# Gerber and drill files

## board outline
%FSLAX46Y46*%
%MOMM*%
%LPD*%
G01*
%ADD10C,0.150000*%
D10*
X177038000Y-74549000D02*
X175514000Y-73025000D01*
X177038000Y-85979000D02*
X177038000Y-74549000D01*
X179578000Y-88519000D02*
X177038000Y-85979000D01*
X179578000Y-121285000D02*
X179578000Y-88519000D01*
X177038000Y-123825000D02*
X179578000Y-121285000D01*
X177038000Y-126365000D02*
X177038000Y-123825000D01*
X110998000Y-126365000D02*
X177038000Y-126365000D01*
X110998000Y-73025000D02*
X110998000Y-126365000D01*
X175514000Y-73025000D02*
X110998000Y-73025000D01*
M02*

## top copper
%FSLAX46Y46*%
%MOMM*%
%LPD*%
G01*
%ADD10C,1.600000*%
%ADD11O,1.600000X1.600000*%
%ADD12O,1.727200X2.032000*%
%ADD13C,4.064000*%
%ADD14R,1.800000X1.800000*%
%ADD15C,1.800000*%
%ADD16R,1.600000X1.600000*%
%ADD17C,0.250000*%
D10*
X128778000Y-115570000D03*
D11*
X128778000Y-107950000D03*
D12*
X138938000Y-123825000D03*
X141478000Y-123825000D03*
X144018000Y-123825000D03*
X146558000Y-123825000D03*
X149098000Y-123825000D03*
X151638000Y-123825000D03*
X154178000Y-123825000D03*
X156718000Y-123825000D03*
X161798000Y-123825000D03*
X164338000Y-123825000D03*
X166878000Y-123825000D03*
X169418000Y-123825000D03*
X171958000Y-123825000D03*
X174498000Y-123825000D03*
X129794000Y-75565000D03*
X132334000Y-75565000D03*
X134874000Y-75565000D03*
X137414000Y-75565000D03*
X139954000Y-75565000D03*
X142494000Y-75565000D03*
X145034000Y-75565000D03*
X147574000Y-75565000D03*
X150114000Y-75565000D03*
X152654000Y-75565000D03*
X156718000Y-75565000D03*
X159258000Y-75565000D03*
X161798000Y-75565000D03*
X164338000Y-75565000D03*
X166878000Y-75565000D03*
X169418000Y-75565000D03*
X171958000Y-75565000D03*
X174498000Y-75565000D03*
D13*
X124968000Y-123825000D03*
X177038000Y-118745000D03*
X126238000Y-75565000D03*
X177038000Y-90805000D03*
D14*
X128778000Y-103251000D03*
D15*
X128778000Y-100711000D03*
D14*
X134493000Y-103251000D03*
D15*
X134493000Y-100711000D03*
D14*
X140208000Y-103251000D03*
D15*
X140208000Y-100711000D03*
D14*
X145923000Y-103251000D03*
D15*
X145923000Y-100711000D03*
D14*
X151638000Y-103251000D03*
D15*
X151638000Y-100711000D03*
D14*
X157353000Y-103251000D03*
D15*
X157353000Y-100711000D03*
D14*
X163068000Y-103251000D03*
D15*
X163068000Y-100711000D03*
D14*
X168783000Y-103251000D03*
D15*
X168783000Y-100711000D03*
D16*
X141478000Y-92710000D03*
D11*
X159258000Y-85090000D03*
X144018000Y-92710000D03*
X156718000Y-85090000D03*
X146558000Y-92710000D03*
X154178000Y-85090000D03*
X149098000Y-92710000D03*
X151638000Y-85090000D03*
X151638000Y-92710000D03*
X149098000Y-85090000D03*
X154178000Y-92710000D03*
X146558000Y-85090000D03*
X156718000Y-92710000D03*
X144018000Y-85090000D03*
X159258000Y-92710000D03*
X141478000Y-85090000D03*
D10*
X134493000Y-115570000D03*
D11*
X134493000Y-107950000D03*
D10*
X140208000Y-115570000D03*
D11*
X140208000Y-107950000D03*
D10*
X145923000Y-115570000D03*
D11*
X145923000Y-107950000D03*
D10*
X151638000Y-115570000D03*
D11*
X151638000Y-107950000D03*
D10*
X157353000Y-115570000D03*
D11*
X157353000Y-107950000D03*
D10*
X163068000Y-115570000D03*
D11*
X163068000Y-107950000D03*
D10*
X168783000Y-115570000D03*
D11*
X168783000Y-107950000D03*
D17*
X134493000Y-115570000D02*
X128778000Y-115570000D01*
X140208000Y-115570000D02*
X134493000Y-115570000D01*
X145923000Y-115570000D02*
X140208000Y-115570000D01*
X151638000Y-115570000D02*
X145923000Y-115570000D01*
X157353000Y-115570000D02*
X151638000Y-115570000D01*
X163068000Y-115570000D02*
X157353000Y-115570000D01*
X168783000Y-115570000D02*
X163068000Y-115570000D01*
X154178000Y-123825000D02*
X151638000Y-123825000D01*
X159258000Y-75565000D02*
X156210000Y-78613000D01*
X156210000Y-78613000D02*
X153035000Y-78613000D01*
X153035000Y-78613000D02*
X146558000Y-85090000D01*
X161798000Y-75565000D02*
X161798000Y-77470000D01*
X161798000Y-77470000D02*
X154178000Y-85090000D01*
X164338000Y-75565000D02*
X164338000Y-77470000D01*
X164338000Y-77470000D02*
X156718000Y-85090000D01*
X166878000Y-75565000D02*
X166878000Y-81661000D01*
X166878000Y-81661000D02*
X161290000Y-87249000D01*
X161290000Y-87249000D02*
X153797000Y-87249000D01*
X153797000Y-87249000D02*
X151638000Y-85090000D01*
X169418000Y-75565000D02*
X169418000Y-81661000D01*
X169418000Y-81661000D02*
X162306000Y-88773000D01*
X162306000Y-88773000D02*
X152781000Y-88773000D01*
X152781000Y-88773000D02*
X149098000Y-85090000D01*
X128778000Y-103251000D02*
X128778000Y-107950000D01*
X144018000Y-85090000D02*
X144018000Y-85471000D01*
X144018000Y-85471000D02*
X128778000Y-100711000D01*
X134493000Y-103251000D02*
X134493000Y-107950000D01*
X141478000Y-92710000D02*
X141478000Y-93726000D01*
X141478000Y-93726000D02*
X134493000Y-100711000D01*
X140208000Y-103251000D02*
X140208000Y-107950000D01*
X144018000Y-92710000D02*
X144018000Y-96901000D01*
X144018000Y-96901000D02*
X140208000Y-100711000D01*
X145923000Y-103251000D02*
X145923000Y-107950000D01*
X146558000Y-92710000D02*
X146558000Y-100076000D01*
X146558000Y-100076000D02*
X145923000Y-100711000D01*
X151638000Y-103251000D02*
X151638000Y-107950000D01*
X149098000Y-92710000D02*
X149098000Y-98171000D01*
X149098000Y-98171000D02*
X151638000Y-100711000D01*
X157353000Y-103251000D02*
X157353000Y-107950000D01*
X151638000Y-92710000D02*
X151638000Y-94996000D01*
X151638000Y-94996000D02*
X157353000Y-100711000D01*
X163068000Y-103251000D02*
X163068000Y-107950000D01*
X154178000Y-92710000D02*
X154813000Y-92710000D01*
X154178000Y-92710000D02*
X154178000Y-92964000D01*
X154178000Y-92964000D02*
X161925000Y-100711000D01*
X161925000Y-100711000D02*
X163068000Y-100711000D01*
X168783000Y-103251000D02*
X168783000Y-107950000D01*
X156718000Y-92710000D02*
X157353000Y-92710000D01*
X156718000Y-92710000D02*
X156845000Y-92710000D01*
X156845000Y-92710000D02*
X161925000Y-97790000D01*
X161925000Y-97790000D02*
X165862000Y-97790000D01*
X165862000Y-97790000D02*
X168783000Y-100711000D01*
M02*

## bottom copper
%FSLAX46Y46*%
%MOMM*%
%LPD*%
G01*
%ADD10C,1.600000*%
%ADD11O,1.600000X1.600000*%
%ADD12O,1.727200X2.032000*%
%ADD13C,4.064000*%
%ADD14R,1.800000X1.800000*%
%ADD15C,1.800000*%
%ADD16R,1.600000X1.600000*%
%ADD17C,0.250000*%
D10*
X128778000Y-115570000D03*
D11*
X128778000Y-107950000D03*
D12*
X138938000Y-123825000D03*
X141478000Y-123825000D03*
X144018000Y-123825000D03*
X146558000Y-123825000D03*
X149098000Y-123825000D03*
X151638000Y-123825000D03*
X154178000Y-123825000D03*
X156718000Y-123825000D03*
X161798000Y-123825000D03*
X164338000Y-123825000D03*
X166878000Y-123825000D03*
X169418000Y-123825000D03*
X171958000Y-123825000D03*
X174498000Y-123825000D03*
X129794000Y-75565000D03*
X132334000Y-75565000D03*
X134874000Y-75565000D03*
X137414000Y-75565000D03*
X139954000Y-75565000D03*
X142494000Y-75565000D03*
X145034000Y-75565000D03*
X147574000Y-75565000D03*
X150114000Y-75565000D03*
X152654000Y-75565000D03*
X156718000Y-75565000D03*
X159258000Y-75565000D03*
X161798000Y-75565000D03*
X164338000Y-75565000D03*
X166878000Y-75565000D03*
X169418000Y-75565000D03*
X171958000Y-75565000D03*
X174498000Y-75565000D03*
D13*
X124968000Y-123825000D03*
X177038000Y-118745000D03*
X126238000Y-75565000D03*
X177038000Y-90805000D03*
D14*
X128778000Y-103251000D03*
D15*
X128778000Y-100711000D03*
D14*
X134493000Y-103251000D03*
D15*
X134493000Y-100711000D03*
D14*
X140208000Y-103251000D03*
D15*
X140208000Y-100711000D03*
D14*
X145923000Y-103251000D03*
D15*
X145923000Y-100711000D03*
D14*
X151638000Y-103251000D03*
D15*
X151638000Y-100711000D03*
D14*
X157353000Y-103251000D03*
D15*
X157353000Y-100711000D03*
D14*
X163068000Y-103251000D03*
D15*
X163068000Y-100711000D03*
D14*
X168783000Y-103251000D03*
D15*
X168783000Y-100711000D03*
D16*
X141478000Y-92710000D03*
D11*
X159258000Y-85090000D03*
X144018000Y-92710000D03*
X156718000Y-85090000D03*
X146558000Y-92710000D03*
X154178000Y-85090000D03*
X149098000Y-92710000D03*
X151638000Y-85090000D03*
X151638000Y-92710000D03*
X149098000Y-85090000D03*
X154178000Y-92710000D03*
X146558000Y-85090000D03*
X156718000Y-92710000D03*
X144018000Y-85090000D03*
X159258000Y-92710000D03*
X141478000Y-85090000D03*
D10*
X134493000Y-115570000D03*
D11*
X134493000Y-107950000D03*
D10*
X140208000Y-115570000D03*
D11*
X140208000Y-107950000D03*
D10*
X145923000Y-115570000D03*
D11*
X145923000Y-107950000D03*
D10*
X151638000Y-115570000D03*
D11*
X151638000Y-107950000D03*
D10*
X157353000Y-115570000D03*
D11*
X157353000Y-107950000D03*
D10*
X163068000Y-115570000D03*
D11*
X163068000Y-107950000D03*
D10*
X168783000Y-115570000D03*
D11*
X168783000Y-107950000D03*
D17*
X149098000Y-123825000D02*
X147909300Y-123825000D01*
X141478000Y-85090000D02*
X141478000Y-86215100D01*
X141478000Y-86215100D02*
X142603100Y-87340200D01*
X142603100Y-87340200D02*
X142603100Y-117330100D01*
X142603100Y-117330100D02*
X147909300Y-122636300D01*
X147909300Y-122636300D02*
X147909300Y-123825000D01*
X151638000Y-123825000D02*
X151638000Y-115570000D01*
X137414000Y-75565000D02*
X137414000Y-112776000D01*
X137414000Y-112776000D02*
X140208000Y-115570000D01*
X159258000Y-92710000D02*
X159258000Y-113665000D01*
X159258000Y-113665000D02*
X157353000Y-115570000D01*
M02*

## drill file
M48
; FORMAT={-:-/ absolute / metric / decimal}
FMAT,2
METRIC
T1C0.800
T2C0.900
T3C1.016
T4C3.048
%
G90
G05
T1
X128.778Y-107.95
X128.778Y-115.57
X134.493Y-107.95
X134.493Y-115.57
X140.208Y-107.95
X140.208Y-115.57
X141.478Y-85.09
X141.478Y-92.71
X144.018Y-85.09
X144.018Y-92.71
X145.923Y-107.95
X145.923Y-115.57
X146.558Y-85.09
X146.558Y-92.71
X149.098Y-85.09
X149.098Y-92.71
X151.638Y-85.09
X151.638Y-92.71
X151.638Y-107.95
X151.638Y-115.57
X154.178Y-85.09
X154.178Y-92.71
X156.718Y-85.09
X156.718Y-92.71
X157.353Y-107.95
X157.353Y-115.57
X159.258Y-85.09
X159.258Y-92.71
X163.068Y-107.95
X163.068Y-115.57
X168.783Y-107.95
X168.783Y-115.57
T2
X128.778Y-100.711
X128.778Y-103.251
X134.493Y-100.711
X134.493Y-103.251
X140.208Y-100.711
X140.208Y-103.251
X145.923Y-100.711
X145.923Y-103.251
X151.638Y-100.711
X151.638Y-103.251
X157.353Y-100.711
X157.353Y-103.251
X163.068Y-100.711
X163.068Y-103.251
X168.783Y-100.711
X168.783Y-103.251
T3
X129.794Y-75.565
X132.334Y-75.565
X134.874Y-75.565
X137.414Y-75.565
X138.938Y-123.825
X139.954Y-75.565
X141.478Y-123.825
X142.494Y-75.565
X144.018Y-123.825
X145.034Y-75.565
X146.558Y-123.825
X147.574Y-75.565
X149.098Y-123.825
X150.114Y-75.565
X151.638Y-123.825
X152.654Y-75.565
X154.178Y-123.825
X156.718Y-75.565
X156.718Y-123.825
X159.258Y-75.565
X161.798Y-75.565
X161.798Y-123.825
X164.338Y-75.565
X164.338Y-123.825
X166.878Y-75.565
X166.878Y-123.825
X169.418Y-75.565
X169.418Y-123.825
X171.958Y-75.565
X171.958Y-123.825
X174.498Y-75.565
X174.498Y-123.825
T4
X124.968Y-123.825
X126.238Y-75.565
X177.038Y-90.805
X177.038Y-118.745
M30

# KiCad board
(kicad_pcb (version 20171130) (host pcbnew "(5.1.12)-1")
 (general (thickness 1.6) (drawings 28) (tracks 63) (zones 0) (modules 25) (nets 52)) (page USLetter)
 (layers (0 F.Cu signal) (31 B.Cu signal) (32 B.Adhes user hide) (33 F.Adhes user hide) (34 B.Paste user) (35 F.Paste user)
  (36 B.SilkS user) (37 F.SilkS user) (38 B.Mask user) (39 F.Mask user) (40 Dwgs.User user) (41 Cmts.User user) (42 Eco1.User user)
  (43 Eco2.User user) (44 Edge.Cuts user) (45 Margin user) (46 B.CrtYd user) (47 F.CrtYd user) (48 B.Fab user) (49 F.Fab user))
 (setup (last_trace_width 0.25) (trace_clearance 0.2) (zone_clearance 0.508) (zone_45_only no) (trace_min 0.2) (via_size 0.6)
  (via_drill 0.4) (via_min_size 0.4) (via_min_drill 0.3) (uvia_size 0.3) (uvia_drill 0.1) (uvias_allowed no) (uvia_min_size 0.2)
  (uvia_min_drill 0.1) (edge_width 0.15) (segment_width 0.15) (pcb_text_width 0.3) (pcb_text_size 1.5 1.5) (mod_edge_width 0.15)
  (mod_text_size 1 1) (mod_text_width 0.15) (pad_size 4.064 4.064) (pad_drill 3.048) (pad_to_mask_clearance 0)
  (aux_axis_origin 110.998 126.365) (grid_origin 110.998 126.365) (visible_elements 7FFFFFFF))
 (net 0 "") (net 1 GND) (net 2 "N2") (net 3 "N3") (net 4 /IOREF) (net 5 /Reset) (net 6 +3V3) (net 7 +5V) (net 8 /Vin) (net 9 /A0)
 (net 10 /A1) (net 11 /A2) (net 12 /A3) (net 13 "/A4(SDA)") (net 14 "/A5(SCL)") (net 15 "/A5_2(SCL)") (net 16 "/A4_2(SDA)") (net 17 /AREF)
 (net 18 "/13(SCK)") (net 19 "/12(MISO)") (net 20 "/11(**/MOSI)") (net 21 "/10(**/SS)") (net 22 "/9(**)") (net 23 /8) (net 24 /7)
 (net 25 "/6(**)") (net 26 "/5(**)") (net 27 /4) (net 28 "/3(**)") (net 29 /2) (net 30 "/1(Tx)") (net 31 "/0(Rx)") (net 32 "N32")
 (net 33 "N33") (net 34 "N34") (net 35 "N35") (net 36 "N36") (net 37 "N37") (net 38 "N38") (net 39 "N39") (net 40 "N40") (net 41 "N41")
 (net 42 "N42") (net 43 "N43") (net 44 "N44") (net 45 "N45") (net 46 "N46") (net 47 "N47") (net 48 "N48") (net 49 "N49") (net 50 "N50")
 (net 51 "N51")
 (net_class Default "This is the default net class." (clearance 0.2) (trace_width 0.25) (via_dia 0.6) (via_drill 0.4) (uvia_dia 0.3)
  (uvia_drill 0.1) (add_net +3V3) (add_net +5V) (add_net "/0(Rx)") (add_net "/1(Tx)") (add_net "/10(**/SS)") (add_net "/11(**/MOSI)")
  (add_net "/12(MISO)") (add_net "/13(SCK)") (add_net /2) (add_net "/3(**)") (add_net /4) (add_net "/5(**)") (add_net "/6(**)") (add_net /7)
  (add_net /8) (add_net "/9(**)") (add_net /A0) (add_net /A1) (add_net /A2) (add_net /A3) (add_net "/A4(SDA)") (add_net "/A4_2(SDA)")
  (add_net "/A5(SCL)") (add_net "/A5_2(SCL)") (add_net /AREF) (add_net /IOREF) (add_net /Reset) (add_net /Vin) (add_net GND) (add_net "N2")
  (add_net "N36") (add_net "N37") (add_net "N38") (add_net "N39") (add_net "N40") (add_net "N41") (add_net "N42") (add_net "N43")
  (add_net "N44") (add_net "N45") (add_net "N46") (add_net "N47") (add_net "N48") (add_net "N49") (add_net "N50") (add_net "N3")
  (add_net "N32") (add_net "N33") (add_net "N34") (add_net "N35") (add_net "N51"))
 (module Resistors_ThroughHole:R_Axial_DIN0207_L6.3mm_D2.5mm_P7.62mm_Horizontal (layer F.Cu) (at 128.778 115.57 90)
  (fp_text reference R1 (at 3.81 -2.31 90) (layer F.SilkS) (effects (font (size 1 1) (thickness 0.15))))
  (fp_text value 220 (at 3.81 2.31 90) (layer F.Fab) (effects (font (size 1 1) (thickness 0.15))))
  (pad 1 thru_hole circle (at 0 0 90) (size 1.6 1.6) (drill 0.8) (layers *.Cu *.Mask) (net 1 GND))
  (pad 2 thru_hole oval (at 7.62 0 90) (size 1.6 1.6) (drill 0.8) (layers *.Cu *.Mask) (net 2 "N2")))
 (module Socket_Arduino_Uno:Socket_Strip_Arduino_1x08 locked (layer F.Cu) (at 138.938 123.825)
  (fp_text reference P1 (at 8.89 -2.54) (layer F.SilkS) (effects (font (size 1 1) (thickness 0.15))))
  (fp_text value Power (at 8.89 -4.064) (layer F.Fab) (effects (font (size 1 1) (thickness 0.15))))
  (pad 1 thru_hole oval (at 0 0) (size 1.7272 2.032) (drill 1.016) (layers *.Cu *.Mask F.SilkS) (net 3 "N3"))
  (pad 2 thru_hole oval (at 2.54 0) (size 1.7272 2.032) (drill 1.016) (layers *.Cu *.Mask F.SilkS) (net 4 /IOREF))
  (pad 3 thru_hole oval (at 5.08 0) (size 1.7272 2.032) (drill 1.016) (layers *.Cu *.Mask F.SilkS) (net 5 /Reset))
  (pad 4 thru_hole oval (at 7.62 0) (size 1.7272 2.032) (drill 1.016) (layers *.Cu *.Mask F.SilkS) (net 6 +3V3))
  (pad 5 thru_hole oval (at 10.16 0) (size 1.7272 2.032) (drill 1.016) (layers *.Cu *.Mask F.SilkS) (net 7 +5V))
  (pad 6 thru_hole oval (at 12.7 0) (size 1.7272 2.032) (drill 1.016) (layers *.Cu *.Mask F.SilkS) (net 1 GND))
  (pad 7 thru_hole oval (at 15.24 0) (size 1.7272 2.032) (drill 1.016) (layers *.Cu *.Mask F.SilkS) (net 1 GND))
  (pad 8 thru_hole oval (at 17.78 0) (size 1.7272 2.032) (drill 1.016) (layers *.Cu *.Mask F.SilkS) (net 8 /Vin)))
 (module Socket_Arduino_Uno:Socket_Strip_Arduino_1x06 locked (layer F.Cu) (at 161.798 123.825)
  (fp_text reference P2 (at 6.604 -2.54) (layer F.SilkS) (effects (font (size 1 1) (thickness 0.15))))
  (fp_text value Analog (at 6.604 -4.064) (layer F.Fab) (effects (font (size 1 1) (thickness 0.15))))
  (pad 1 thru_hole oval (at 0 0) (size 1.7272 2.032) (drill 1.016) (layers *.Cu *.Mask F.SilkS) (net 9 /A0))
  (pad 2 thru_hole oval (at 2.54 0) (size 1.7272 2.032) (drill 1.016) (layers *.Cu *.Mask F.SilkS) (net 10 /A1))
  (pad 3 thru_hole oval (at 5.08 0) (size 1.7272 2.032) (drill 1.016) (layers *.Cu *.Mask F.SilkS) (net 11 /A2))
  (pad 4 thru_hole oval (at 7.62 0) (size 1.7272 2.032) (drill 1.016) (layers *.Cu *.Mask F.SilkS) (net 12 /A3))
  (pad 5 thru_hole oval (at 10.16 0) (size 1.7272 2.032) (drill 1.016) (layers *.Cu *.Mask F.SilkS) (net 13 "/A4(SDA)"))
  (pad 6 thru_hole oval (at 12.7 0) (size 1.7272 2.032) (drill 1.016) (layers *.Cu *.Mask F.SilkS) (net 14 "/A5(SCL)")))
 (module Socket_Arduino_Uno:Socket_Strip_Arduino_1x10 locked (layer F.Cu) (at 129.794 75.565)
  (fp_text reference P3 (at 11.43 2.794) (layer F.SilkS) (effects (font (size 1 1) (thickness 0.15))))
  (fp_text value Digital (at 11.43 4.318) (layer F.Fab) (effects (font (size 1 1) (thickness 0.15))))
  (pad 1 thru_hole oval (at 0 0) (size 1.7272 2.032) (drill 1.016) (layers *.Cu *.Mask F.SilkS) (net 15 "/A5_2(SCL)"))
  (pad 2 thru_hole oval (at 2.54 0) (size 1.7272 2.032) (drill 1.016) (layers *.Cu *.Mask F.SilkS) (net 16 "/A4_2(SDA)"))
  (pad 3 thru_hole oval (at 5.08 0) (size 1.7272 2.032) (drill 1.016) (layers *.Cu *.Mask F.SilkS) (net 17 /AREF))
  (pad 4 thru_hole oval (at 7.62 0) (size 1.7272 2.032) (drill 1.016) (layers *.Cu *.Mask F.SilkS) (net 1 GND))
  (pad 5 thru_hole oval (at 10.16 0) (size 1.7272 2.032) (drill 1.016) (layers *.Cu *.Mask F.SilkS) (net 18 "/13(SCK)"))
  (pad 6 thru_hole oval (at 12.7 0) (size 1.7272 2.032) (drill 1.016) (layers *.Cu *.Mask F.SilkS) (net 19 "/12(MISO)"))
  (pad 7 thru_hole oval (at 15.24 0) (size 1.7272 2.032) (drill 1.016) (layers *.Cu *.Mask F.SilkS) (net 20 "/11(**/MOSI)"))
  (pad 8 thru_hole oval (at 17.78 0) (size 1.7272 2.032) (drill 1.016) (layers *.Cu *.Mask F.SilkS) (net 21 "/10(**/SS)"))
  (pad 9 thru_hole oval (at 20.32 0) (size 1.7272 2.032) (drill 1.016) (layers *.Cu *.Mask F.SilkS) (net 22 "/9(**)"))
  (pad 10 thru_hole oval (at 22.86 0) (size 1.7272 2.032) (drill 1.016) (layers *.Cu *.Mask F.SilkS) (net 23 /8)))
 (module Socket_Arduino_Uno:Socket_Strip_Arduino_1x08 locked (layer F.Cu) (at 156.718 75.565)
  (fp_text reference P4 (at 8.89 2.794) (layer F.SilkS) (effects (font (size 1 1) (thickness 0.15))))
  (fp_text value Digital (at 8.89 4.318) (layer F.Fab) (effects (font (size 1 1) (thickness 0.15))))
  (pad 1 thru_hole oval (at 0 0) (size 1.7272 2.032) (drill 1.016) (layers *.Cu *.Mask F.SilkS) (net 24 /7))
  (pad 2 thru_hole oval (at 2.54 0) (size 1.7272 2.032) (drill 1.016) (layers *.Cu *.Mask F.SilkS) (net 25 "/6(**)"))
  (pad 3 thru_hole oval (at 5.08 0) (size 1.7272 2.032) (drill 1.016) (layers *.Cu *.Mask F.SilkS) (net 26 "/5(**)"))
  (pad 4 thru_hole oval (at 7.62 0) (size 1.7272 2.032) (drill 1.016) (layers *.Cu *.Mask F.SilkS) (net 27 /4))
  (pad 5 thru_hole oval (at 10.16 0) (size 1.7272 2.032) (drill 1.016) (layers *.Cu *.Mask F.SilkS) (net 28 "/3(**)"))
  (pad 6 thru_hole oval (at 12.7 0) (size 1.7272 2.032) (drill 1.016) (layers *.Cu *.Mask F.SilkS) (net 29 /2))
  (pad 7 thru_hole oval (at 15.24 0) (size 1.7272 2.032) (drill 1.016) (layers *.Cu *.Mask F.SilkS) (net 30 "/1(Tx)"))
  (pad 8 thru_hole oval (at 17.78 0) (size 1.7272 2.032) (drill 1.016) (layers *.Cu *.Mask F.SilkS) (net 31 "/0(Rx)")))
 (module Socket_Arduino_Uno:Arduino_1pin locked (layer F.Cu) (at 124.968 123.825)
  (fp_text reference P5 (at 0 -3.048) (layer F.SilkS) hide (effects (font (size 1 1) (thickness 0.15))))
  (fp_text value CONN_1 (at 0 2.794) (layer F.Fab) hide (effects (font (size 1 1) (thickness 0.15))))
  (pad 1 thru_hole circle (at 0 0) (size 4.064 4.064) (drill 3.048) (layers *.Cu *.Mask F.SilkS) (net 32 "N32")))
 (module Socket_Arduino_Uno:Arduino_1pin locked (layer F.Cu) (at 177.038 118.745)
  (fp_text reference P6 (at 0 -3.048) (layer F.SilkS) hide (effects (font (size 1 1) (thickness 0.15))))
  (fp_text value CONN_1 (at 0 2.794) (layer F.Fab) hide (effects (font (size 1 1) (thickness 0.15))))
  (pad 1 thru_hole circle (at 0 0) (size 4.064 4.064) (drill 3.048) (layers *.Cu *.Mask F.SilkS) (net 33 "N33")))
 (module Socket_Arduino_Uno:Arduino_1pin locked (layer F.Cu) (at 126.238 75.565)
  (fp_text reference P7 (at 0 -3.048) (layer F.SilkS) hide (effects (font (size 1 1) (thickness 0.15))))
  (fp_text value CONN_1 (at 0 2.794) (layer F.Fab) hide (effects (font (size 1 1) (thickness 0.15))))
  (pad 1 thru_hole circle (at 0 0) (size 4.064 4.064) (drill 3.048) (layers *.Cu *.Mask F.SilkS) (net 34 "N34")))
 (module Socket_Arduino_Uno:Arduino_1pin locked (layer F.Cu) (at 177.038 90.805)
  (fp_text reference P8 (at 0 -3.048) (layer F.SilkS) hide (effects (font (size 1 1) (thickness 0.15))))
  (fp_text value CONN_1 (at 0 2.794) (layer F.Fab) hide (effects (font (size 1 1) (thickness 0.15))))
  (pad 1 thru_hole circle (at 0 0) (size 4.064 4.064) (drill 3.048) (layers *.Cu *.Mask F.SilkS) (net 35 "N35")))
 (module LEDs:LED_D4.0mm (layer F.Cu) (at 128.778 103.251 90)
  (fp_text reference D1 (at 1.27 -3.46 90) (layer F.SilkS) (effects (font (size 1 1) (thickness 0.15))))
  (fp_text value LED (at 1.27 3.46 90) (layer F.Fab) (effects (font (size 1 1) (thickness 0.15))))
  (pad 1 thru_hole rect (at 0 0 90) (size 1.8 1.8) (drill 0.9) (layers *.Cu *.Mask) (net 2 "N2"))
  (pad 2 thru_hole circle (at 2.54 0 90) (size 1.8 1.8) (drill 0.9) (layers *.Cu *.Mask) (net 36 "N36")))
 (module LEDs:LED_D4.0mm (layer F.Cu) (at 134.493 103.251 90)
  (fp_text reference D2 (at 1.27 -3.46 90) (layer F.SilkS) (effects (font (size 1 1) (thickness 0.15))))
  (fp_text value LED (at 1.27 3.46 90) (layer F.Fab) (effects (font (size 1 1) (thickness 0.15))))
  (pad 1 thru_hole rect (at 0 0 90) (size 1.8 1.8) (drill 0.9) (layers *.Cu *.Mask) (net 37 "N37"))
  (pad 2 thru_hole circle (at 2.54 0 90) (size 1.8 1.8) (drill 0.9) (layers *.Cu *.Mask) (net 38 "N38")))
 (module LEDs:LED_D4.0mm (layer F.Cu) (at 140.208 103.251 90)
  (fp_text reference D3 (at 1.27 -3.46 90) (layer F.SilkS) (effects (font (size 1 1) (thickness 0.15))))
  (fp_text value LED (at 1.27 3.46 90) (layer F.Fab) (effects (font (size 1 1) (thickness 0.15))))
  (pad 1 thru_hole rect (at 0 0 90) (size 1.8 1.8) (drill 0.9) (layers *.Cu *.Mask) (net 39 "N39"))
  (pad 2 thru_hole circle (at 2.54 0 90) (size 1.8 1.8) (drill 0.9) (layers *.Cu *.Mask) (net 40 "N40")))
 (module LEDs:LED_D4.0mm (layer F.Cu) (at 145.923 103.251 90)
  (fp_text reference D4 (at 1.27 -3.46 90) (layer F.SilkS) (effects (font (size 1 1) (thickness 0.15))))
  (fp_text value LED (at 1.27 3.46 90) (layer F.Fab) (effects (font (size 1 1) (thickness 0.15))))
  (pad 1 thru_hole rect (at 0 0 90) (size 1.8 1.8) (drill 0.9) (layers *.Cu *.Mask) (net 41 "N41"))
  (pad 2 thru_hole circle (at 2.54 0 90) (size 1.8 1.8) (drill 0.9) (layers *.Cu *.Mask) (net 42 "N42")))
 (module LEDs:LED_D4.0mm (layer F.Cu) (at 151.638 103.251 90)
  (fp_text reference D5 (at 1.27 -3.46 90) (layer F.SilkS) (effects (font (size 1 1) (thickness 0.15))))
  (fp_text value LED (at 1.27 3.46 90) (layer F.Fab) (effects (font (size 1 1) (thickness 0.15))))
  (pad 1 thru_hole rect (at 0 0 90) (size 1.8 1.8) (drill 0.9) (layers *.Cu *.Mask) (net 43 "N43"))
  (pad 2 thru_hole circle (at 2.54 0 90) (size 1.8 1.8) (drill 0.9) (layers *.Cu *.Mask) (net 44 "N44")))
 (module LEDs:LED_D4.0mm (layer F.Cu) (at 157.353 103.251 90)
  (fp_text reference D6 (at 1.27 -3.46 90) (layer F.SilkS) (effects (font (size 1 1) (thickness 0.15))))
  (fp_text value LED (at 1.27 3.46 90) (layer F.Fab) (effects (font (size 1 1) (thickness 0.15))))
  (pad 1 thru_hole rect (at 0 0 90) (size 1.8 1.8) (drill 0.9) (layers *.Cu *.Mask) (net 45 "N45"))
  (pad 2 thru_hole circle (at 2.54 0 90) (size 1.8 1.8) (drill 0.9) (layers *.Cu *.Mask) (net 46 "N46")))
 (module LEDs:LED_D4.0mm (layer F.Cu) (at 163.068 103.251 90)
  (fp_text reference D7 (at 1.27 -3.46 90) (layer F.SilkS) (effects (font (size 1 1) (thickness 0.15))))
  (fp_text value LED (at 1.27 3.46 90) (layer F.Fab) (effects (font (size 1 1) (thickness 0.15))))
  (pad 1 thru_hole rect (at 0 0 90) (size 1.8 1.8) (drill 0.9) (layers *.Cu *.Mask) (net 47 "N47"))
  (pad 2 thru_hole circle (at 2.54 0 90) (size 1.8 1.8) (drill 0.9) (layers *.Cu *.Mask) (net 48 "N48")))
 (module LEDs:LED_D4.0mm (layer F.Cu) (at 168.783 103.251 90)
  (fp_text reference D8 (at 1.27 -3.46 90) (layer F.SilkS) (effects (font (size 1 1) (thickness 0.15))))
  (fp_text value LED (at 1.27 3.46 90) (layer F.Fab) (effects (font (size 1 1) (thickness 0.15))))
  (pad 1 thru_hole rect (at 0 0 90) (size 1.8 1.8) (drill 0.9) (layers *.Cu *.Mask) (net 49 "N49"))
  (pad 2 thru_hole circle (at 2.54 0 90) (size 1.8 1.8) (drill 0.9) (layers *.Cu *.Mask) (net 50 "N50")))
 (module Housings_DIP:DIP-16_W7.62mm (layer F.Cu) (at 141.478 92.71 90)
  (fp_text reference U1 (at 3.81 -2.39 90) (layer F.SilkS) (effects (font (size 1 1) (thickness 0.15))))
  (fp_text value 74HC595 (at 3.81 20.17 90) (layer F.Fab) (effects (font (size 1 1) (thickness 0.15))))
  (pad 1 thru_hole rect (at 0 0 90) (size 1.6 1.6) (drill 0.8) (layers *.Cu *.Mask) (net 38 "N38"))
  (pad 9 thru_hole oval (at 7.62 17.78 90) (size 1.6 1.6) (drill 0.8) (layers *.Cu *.Mask) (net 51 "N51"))
  (pad 2 thru_hole oval (at 0 2.54 90) (size 1.6 1.6) (drill 0.8) (layers *.Cu *.Mask) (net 40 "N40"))
  (pad 10 thru_hole oval (at 7.62 15.24 90) (size 1.6 1.6) (drill 0.8) (layers *.Cu *.Mask) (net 27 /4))
  (pad 3 thru_hole oval (at 0 5.08 90) (size 1.6 1.6) (drill 0.8) (layers *.Cu *.Mask) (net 42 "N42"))
  (pad 11 thru_hole oval (at 7.62 12.7 90) (size 1.6 1.6) (drill 0.8) (layers *.Cu *.Mask) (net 26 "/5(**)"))
  (pad 4 thru_hole oval (at 0 7.62 90) (size 1.6 1.6) (drill 0.8) (layers *.Cu *.Mask) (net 44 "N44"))
  (pad 12 thru_hole oval (at 7.62 10.16 90) (size 1.6 1.6) (drill 0.8) (layers *.Cu *.Mask) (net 28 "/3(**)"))
  (pad 5 thru_hole oval (at 0 10.16 90) (size 1.6 1.6) (drill 0.8) (layers *.Cu *.Mask) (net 46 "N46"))
  (pad 13 thru_hole oval (at 7.62 7.62 90) (size 1.6 1.6) (drill 0.8) (layers *.Cu *.Mask) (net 29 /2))
  (pad 6 thru_hole oval (at 0 12.7 90) (size 1.6 1.6) (drill 0.8) (layers *.Cu *.Mask) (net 48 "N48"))
  (pad 14 thru_hole oval (at 7.62 5.08 90) (size 1.6 1.6) (drill 0.8) (layers *.Cu *.Mask) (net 25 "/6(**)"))
  (pad 7 thru_hole oval (at 0 15.24 90) (size 1.6 1.6) (drill 0.8) (layers *.Cu *.Mask) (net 50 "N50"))
  (pad 15 thru_hole oval (at 7.62 2.54 90) (size 1.6 1.6) (drill 0.8) (layers *.Cu *.Mask) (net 36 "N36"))
  (pad 8 thru_hole oval (at 0 17.78 90) (size 1.6 1.6) (drill 0.8) (layers *.Cu *.Mask) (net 1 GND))
  (pad 16 thru_hole oval (at 7.62 0 90) (size 1.6 1.6) (drill 0.8) (layers *.Cu *.Mask) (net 7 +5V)))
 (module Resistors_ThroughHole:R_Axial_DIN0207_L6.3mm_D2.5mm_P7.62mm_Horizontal (layer F.Cu) (at 134.493 115.57 90)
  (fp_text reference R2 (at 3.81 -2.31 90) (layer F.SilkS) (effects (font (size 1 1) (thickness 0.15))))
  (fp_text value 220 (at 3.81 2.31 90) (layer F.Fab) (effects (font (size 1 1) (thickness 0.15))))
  (pad 1 thru_hole circle (at 0 0 90) (size 1.6 1.6) (drill 0.8) (layers *.Cu *.Mask) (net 1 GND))
  (pad 2 thru_hole oval (at 7.62 0 90) (size 1.6 1.6) (drill 0.8) (layers *.Cu *.Mask) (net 37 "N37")))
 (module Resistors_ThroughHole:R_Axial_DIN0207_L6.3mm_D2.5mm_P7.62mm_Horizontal (layer F.Cu) (at 140.208 115.57 90)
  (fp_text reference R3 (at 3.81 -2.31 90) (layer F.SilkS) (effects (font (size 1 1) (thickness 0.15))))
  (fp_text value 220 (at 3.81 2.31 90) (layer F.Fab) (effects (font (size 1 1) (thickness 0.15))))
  (pad 1 thru_hole circle (at 0 0 90) (size 1.6 1.6) (drill 0.8) (layers *.Cu *.Mask) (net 1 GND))
  (pad 2 thru_hole oval (at 7.62 0 90) (size 1.6 1.6) (drill 0.8) (layers *.Cu *.Mask) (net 39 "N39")))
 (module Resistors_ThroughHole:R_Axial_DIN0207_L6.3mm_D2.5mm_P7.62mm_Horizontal (layer F.Cu) (at 145.923 115.57 90)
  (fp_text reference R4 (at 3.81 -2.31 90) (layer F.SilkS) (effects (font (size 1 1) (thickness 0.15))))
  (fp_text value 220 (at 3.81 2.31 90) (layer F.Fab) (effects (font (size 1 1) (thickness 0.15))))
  (pad 1 thru_hole circle (at 0 0 90) (size 1.6 1.6) (drill 0.8) (layers *.Cu *.Mask) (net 1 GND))
  (pad 2 thru_hole oval (at 7.62 0 90) (size 1.6 1.6) (drill 0.8) (layers *.Cu *.Mask) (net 41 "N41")))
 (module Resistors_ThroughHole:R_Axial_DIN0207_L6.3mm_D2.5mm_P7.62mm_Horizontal (layer F.Cu) (at 151.638 115.57 90)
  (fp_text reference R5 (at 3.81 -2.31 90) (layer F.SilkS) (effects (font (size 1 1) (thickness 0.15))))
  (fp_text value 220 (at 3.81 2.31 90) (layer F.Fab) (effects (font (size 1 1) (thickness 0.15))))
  (pad 1 thru_hole circle (at 0 0 90) (size 1.6 1.6) (drill 0.8) (layers *.Cu *.Mask) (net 1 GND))
  (pad 2 thru_hole oval (at 7.62 0 90) (size 1.6 1.6) (drill 0.8) (layers *.Cu *.Mask) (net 43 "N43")))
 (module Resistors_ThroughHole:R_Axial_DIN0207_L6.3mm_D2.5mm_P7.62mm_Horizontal (layer F.Cu) (at 157.353 115.57 90)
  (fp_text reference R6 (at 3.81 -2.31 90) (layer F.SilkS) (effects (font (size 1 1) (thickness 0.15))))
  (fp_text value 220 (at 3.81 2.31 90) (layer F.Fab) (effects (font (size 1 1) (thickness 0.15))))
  (pad 1 thru_hole circle (at 0 0 90) (size 1.6 1.6) (drill 0.8) (layers *.Cu *.Mask) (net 1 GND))
  (pad 2 thru_hole oval (at 7.62 0 90) (size 1.6 1.6) (drill 0.8) (layers *.Cu *.Mask) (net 45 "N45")))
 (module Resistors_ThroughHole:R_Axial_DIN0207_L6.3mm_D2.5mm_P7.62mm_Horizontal (layer F.Cu) (at 163.068 115.57 90)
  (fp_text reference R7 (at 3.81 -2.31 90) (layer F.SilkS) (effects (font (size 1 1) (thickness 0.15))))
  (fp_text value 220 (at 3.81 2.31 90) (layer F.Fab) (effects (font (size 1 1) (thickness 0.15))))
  (pad 1 thru_hole circle (at 0 0 90) (size 1.6 1.6) (drill 0.8) (layers *.Cu *.Mask) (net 1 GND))
  (pad 2 thru_hole oval (at 7.62 0 90) (size 1.6 1.6) (drill 0.8) (layers *.Cu *.Mask) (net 47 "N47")))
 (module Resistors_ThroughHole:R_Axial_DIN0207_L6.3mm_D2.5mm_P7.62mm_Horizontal (layer F.Cu) (at 168.783 115.57 90)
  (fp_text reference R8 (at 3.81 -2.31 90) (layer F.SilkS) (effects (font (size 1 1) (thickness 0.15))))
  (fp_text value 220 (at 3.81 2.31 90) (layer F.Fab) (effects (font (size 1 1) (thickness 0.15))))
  (pad 1 thru_hole circle (at 0 0 90) (size 1.6 1.6) (drill 0.8) (layers *.Cu *.Mask) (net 1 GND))
  (pad 2 thru_hole oval (at 7.62 0 90) (size 1.6 1.6) (drill 0.8) (layers *.Cu *.Mask) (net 49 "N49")))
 (gr_line (start 177.038 74.549) (end 175.514 73.025) (angle 90) (layer Edge.Cuts) (width 0.15))
 (gr_line (start 177.038 85.979) (end 177.038 74.549) (angle 90) (layer Edge.Cuts) (width 0.15))
 (gr_line (start 179.578 88.519) (end 177.038 85.979) (angle 90) (layer Edge.Cuts) (width 0.15))
 (gr_line (start 179.578 121.285) (end 179.578 88.519) (angle 90) (layer Edge.Cuts) (width 0.15))
 (gr_line (start 177.038 123.825) (end 179.578 121.285) (angle 90) (layer Edge.Cuts) (width 0.15))
 (gr_line (start 177.038 126.365) (end 177.038 123.825) (angle 90) (layer Edge.Cuts) (width 0.15))
 (gr_line (start 110.998 126.365) (end 177.038 126.365) (angle 90) (layer Edge.Cuts) (width 0.15))
 (gr_line (start 110.998 73.025) (end 110.998 126.365) (angle 90) (layer Edge.Cuts) (width 0.15))
 (gr_line (start 175.514 73.025) (end 110.998 73.025) (angle 90) (layer Edge.Cuts) (width 0.15))
 (segment (start 149.098 123.825) (end 147.9093 123.825) (width 0.25) (layer B.Cu) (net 7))
 (segment (start 141.478 85.09) (end 141.478 86.2151) (width 0.25) (layer B.Cu) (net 7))
 (segment (start 141.478 86.2151) (end 142.6031 87.3402) (width 0.25) (layer B.Cu) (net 7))
 (segment (start 142.6031 87.3402) (end 142.6031 117.3301) (width 0.25) (layer B.Cu) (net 7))
 (segment (start 142.6031 117.3301) (end 147.9093 122.6363) (width 0.25) (layer B.Cu) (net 7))
 (segment (start 147.9093 122.6363) (end 147.9093 123.825) (width 0.25) (layer B.Cu) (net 7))
 (segment (start 134.493 115.57) (end 128.778 115.57) (width 0.25) (layer F.Cu) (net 1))
 (segment (start 140.208 115.57) (end 134.493 115.57) (width 0.25) (layer F.Cu) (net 1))
 (segment (start 145.923 115.57) (end 140.208 115.57) (width 0.25) (layer F.Cu) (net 1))
 (segment (start 151.638 115.57) (end 145.923 115.57) (width 0.25) (layer F.Cu) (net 1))
 (segment (start 157.353 115.57) (end 151.638 115.57) (width 0.25) (layer F.Cu) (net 1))
 (segment (start 163.068 115.57) (end 157.353 115.57) (width 0.25) (layer F.Cu) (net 1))
 (segment (start 168.783 115.57) (end 163.068 115.57) (width 0.25) (layer F.Cu) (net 1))
 (segment (start 151.638 123.825) (end 151.638 115.57) (width 0.25) (layer B.Cu) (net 1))
 (segment (start 154.178 123.825) (end 151.638 123.825) (width 0.25) (layer F.Cu) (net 1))
 (segment (start 137.414 75.565) (end 137.414 112.776) (width 0.25) (layer B.Cu) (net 1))
 (segment (start 137.414 112.776) (end 140.208 115.57) (width 0.25) (layer B.Cu) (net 1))
 (segment (start 159.258 92.71) (end 159.258 113.665) (width 0.25) (layer B.Cu) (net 1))
 (segment (start 159.258 113.665) (end 157.353 115.57) (width 0.25) (layer B.Cu) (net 1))
 (segment (start 159.258 75.565) (end 156.21 78.613) (width 0.25) (layer F.Cu) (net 25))
 (segment (start 156.21 78.613) (end 153.035 78.613) (width 0.25) (layer F.Cu) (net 25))
 (segment (start 153.035 78.613) (end 146.558 85.09) (width 0.25) (layer F.Cu) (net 25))
 (segment (start 161.798 75.565) (end 161.798 77.47) (width 0.25) (layer F.Cu) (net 26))
 (segment (start 161.798 77.47) (end 154.178 85.09) (width 0.25) (layer F.Cu) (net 26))
 (segment (start 164.338 75.565) (end 164.338 77.47) (width 0.25) (layer F.Cu) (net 27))
 (segment (start 164.338 77.47) (end 156.718 85.09) (width 0.25) (layer F.Cu) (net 27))
 (segment (start 166.878 75.565) (end 166.878 81.661) (width 0.25) (layer F.Cu) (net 28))
 (segment (start 166.878 81.661) (end 161.29 87.249) (width 0.25) (layer F.Cu) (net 28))
 (segment (start 161.29 87.249) (end 153.797 87.249) (width 0.25) (layer F.Cu) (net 28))
 (segment (start 153.797 87.249) (end 151.638 85.09) (width 0.25) (layer F.Cu) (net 28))
 (segment (start 169.418 75.565) (end 169.418 81.661) (width 0.25) (layer F.Cu) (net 29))
 (segment (start 169.418 81.661) (end 162.306 88.773) (width 0.25) (layer F.Cu) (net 29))
 (segment (start 162.306 88.773) (end 152.781 88.773) (width 0.25) (layer F.Cu) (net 29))
 (segment (start 152.781 88.773) (end 149.098 85.09) (width 0.25) (layer F.Cu) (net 29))
 (segment (start 128.778 103.251) (end 128.778 107.95) (width 0.25) (layer F.Cu) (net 2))
 (segment (start 144.018 85.09) (end 144.018 85.471) (width 0.25) (layer F.Cu) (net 36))
 (segment (start 144.018 85.471) (end 128.778 100.711) (width 0.25) (layer F.Cu) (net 36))
 (segment (start 134.493 103.251) (end 134.493 107.95) (width 0.25) (layer F.Cu) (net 37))
 (segment (start 141.478 92.71) (end 141.478 93.726) (width 0.25) (layer F.Cu) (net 38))
 (segment (start 141.478 93.726) (end 134.493 100.711) (width 0.25) (layer F.Cu) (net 38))
 (segment (start 140.208 103.251) (end 140.208 107.95) (width 0.25) (layer F.Cu) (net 39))
 (segment (start 144.018 92.71) (end 144.018 96.901) (width 0.25) (layer F.Cu) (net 40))
 (segment (start 144.018 96.901) (end 140.208 100.711) (width 0.25) (layer F.Cu) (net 40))
 (segment (start 145.923 103.251) (end 145.923 107.95) (width 0.25) (layer F.Cu) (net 41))
 (segment (start 146.558 92.71) (end 146.558 100.076) (width 0.25) (layer F.Cu) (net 42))
 (segment (start 146.558 100.076) (end 145.923 100.711) (width 0.25) (layer F.Cu) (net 42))
 (segment (start 151.638 103.251) (end 151.638 107.95) (width 0.25) (layer F.Cu) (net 43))
 (segment (start 149.098 92.71) (end 149.098 98.171) (width 0.25) (layer F.Cu) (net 44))
 (segment (start 149.098 98.171) (end 151.638 100.711) (width 0.25) (layer F.Cu) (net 44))
 (segment (start 157.353 103.251) (end 157.353 107.95) (width 0.25) (layer F.Cu) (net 45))
 (segment (start 151.638 92.71) (end 151.638 94.996) (width 0.25) (layer F.Cu) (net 46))
 (segment (start 151.638 94.996) (end 157.353 100.711) (width 0.25) (layer F.Cu) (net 46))
 (segment (start 163.068 103.251) (end 163.068 107.95) (width 0.25) (layer F.Cu) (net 47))
 (segment (start 154.178 92.71) (end 154.813 92.71) (width 0.25) (layer F.Cu) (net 48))
 (segment (start 154.178 92.71) (end 154.178 92.964) (width 0.25) (layer F.Cu) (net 48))
 (segment (start 154.178 92.964) (end 161.925 100.711) (width 0.25) (layer F.Cu) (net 48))
 (segment (start 161.925 100.711) (end 163.068 100.711) (width 0.25) (layer F.Cu) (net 48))
 (segment (start 168.783 103.251) (end 168.783 107.95) (width 0.25) (layer F.Cu) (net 49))
 (segment (start 156.718 92.71) (end 157.353 92.71) (width 0.25) (layer F.Cu) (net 50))
 (segment (start 156.718 92.71) (end 156.845 92.71) (width 0.25) (layer F.Cu) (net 50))
 (segment (start 156.845 92.71) (end 161.925 97.79) (width 0.25) (layer F.Cu) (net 50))
 (segment (start 161.925 97.79) (end 165.862 97.79) (width 0.25) (layer F.Cu) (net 50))
 (segment (start 165.862 97.79) (end 168.783 100.711) (width 0.25) (layer F.Cu) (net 50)))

